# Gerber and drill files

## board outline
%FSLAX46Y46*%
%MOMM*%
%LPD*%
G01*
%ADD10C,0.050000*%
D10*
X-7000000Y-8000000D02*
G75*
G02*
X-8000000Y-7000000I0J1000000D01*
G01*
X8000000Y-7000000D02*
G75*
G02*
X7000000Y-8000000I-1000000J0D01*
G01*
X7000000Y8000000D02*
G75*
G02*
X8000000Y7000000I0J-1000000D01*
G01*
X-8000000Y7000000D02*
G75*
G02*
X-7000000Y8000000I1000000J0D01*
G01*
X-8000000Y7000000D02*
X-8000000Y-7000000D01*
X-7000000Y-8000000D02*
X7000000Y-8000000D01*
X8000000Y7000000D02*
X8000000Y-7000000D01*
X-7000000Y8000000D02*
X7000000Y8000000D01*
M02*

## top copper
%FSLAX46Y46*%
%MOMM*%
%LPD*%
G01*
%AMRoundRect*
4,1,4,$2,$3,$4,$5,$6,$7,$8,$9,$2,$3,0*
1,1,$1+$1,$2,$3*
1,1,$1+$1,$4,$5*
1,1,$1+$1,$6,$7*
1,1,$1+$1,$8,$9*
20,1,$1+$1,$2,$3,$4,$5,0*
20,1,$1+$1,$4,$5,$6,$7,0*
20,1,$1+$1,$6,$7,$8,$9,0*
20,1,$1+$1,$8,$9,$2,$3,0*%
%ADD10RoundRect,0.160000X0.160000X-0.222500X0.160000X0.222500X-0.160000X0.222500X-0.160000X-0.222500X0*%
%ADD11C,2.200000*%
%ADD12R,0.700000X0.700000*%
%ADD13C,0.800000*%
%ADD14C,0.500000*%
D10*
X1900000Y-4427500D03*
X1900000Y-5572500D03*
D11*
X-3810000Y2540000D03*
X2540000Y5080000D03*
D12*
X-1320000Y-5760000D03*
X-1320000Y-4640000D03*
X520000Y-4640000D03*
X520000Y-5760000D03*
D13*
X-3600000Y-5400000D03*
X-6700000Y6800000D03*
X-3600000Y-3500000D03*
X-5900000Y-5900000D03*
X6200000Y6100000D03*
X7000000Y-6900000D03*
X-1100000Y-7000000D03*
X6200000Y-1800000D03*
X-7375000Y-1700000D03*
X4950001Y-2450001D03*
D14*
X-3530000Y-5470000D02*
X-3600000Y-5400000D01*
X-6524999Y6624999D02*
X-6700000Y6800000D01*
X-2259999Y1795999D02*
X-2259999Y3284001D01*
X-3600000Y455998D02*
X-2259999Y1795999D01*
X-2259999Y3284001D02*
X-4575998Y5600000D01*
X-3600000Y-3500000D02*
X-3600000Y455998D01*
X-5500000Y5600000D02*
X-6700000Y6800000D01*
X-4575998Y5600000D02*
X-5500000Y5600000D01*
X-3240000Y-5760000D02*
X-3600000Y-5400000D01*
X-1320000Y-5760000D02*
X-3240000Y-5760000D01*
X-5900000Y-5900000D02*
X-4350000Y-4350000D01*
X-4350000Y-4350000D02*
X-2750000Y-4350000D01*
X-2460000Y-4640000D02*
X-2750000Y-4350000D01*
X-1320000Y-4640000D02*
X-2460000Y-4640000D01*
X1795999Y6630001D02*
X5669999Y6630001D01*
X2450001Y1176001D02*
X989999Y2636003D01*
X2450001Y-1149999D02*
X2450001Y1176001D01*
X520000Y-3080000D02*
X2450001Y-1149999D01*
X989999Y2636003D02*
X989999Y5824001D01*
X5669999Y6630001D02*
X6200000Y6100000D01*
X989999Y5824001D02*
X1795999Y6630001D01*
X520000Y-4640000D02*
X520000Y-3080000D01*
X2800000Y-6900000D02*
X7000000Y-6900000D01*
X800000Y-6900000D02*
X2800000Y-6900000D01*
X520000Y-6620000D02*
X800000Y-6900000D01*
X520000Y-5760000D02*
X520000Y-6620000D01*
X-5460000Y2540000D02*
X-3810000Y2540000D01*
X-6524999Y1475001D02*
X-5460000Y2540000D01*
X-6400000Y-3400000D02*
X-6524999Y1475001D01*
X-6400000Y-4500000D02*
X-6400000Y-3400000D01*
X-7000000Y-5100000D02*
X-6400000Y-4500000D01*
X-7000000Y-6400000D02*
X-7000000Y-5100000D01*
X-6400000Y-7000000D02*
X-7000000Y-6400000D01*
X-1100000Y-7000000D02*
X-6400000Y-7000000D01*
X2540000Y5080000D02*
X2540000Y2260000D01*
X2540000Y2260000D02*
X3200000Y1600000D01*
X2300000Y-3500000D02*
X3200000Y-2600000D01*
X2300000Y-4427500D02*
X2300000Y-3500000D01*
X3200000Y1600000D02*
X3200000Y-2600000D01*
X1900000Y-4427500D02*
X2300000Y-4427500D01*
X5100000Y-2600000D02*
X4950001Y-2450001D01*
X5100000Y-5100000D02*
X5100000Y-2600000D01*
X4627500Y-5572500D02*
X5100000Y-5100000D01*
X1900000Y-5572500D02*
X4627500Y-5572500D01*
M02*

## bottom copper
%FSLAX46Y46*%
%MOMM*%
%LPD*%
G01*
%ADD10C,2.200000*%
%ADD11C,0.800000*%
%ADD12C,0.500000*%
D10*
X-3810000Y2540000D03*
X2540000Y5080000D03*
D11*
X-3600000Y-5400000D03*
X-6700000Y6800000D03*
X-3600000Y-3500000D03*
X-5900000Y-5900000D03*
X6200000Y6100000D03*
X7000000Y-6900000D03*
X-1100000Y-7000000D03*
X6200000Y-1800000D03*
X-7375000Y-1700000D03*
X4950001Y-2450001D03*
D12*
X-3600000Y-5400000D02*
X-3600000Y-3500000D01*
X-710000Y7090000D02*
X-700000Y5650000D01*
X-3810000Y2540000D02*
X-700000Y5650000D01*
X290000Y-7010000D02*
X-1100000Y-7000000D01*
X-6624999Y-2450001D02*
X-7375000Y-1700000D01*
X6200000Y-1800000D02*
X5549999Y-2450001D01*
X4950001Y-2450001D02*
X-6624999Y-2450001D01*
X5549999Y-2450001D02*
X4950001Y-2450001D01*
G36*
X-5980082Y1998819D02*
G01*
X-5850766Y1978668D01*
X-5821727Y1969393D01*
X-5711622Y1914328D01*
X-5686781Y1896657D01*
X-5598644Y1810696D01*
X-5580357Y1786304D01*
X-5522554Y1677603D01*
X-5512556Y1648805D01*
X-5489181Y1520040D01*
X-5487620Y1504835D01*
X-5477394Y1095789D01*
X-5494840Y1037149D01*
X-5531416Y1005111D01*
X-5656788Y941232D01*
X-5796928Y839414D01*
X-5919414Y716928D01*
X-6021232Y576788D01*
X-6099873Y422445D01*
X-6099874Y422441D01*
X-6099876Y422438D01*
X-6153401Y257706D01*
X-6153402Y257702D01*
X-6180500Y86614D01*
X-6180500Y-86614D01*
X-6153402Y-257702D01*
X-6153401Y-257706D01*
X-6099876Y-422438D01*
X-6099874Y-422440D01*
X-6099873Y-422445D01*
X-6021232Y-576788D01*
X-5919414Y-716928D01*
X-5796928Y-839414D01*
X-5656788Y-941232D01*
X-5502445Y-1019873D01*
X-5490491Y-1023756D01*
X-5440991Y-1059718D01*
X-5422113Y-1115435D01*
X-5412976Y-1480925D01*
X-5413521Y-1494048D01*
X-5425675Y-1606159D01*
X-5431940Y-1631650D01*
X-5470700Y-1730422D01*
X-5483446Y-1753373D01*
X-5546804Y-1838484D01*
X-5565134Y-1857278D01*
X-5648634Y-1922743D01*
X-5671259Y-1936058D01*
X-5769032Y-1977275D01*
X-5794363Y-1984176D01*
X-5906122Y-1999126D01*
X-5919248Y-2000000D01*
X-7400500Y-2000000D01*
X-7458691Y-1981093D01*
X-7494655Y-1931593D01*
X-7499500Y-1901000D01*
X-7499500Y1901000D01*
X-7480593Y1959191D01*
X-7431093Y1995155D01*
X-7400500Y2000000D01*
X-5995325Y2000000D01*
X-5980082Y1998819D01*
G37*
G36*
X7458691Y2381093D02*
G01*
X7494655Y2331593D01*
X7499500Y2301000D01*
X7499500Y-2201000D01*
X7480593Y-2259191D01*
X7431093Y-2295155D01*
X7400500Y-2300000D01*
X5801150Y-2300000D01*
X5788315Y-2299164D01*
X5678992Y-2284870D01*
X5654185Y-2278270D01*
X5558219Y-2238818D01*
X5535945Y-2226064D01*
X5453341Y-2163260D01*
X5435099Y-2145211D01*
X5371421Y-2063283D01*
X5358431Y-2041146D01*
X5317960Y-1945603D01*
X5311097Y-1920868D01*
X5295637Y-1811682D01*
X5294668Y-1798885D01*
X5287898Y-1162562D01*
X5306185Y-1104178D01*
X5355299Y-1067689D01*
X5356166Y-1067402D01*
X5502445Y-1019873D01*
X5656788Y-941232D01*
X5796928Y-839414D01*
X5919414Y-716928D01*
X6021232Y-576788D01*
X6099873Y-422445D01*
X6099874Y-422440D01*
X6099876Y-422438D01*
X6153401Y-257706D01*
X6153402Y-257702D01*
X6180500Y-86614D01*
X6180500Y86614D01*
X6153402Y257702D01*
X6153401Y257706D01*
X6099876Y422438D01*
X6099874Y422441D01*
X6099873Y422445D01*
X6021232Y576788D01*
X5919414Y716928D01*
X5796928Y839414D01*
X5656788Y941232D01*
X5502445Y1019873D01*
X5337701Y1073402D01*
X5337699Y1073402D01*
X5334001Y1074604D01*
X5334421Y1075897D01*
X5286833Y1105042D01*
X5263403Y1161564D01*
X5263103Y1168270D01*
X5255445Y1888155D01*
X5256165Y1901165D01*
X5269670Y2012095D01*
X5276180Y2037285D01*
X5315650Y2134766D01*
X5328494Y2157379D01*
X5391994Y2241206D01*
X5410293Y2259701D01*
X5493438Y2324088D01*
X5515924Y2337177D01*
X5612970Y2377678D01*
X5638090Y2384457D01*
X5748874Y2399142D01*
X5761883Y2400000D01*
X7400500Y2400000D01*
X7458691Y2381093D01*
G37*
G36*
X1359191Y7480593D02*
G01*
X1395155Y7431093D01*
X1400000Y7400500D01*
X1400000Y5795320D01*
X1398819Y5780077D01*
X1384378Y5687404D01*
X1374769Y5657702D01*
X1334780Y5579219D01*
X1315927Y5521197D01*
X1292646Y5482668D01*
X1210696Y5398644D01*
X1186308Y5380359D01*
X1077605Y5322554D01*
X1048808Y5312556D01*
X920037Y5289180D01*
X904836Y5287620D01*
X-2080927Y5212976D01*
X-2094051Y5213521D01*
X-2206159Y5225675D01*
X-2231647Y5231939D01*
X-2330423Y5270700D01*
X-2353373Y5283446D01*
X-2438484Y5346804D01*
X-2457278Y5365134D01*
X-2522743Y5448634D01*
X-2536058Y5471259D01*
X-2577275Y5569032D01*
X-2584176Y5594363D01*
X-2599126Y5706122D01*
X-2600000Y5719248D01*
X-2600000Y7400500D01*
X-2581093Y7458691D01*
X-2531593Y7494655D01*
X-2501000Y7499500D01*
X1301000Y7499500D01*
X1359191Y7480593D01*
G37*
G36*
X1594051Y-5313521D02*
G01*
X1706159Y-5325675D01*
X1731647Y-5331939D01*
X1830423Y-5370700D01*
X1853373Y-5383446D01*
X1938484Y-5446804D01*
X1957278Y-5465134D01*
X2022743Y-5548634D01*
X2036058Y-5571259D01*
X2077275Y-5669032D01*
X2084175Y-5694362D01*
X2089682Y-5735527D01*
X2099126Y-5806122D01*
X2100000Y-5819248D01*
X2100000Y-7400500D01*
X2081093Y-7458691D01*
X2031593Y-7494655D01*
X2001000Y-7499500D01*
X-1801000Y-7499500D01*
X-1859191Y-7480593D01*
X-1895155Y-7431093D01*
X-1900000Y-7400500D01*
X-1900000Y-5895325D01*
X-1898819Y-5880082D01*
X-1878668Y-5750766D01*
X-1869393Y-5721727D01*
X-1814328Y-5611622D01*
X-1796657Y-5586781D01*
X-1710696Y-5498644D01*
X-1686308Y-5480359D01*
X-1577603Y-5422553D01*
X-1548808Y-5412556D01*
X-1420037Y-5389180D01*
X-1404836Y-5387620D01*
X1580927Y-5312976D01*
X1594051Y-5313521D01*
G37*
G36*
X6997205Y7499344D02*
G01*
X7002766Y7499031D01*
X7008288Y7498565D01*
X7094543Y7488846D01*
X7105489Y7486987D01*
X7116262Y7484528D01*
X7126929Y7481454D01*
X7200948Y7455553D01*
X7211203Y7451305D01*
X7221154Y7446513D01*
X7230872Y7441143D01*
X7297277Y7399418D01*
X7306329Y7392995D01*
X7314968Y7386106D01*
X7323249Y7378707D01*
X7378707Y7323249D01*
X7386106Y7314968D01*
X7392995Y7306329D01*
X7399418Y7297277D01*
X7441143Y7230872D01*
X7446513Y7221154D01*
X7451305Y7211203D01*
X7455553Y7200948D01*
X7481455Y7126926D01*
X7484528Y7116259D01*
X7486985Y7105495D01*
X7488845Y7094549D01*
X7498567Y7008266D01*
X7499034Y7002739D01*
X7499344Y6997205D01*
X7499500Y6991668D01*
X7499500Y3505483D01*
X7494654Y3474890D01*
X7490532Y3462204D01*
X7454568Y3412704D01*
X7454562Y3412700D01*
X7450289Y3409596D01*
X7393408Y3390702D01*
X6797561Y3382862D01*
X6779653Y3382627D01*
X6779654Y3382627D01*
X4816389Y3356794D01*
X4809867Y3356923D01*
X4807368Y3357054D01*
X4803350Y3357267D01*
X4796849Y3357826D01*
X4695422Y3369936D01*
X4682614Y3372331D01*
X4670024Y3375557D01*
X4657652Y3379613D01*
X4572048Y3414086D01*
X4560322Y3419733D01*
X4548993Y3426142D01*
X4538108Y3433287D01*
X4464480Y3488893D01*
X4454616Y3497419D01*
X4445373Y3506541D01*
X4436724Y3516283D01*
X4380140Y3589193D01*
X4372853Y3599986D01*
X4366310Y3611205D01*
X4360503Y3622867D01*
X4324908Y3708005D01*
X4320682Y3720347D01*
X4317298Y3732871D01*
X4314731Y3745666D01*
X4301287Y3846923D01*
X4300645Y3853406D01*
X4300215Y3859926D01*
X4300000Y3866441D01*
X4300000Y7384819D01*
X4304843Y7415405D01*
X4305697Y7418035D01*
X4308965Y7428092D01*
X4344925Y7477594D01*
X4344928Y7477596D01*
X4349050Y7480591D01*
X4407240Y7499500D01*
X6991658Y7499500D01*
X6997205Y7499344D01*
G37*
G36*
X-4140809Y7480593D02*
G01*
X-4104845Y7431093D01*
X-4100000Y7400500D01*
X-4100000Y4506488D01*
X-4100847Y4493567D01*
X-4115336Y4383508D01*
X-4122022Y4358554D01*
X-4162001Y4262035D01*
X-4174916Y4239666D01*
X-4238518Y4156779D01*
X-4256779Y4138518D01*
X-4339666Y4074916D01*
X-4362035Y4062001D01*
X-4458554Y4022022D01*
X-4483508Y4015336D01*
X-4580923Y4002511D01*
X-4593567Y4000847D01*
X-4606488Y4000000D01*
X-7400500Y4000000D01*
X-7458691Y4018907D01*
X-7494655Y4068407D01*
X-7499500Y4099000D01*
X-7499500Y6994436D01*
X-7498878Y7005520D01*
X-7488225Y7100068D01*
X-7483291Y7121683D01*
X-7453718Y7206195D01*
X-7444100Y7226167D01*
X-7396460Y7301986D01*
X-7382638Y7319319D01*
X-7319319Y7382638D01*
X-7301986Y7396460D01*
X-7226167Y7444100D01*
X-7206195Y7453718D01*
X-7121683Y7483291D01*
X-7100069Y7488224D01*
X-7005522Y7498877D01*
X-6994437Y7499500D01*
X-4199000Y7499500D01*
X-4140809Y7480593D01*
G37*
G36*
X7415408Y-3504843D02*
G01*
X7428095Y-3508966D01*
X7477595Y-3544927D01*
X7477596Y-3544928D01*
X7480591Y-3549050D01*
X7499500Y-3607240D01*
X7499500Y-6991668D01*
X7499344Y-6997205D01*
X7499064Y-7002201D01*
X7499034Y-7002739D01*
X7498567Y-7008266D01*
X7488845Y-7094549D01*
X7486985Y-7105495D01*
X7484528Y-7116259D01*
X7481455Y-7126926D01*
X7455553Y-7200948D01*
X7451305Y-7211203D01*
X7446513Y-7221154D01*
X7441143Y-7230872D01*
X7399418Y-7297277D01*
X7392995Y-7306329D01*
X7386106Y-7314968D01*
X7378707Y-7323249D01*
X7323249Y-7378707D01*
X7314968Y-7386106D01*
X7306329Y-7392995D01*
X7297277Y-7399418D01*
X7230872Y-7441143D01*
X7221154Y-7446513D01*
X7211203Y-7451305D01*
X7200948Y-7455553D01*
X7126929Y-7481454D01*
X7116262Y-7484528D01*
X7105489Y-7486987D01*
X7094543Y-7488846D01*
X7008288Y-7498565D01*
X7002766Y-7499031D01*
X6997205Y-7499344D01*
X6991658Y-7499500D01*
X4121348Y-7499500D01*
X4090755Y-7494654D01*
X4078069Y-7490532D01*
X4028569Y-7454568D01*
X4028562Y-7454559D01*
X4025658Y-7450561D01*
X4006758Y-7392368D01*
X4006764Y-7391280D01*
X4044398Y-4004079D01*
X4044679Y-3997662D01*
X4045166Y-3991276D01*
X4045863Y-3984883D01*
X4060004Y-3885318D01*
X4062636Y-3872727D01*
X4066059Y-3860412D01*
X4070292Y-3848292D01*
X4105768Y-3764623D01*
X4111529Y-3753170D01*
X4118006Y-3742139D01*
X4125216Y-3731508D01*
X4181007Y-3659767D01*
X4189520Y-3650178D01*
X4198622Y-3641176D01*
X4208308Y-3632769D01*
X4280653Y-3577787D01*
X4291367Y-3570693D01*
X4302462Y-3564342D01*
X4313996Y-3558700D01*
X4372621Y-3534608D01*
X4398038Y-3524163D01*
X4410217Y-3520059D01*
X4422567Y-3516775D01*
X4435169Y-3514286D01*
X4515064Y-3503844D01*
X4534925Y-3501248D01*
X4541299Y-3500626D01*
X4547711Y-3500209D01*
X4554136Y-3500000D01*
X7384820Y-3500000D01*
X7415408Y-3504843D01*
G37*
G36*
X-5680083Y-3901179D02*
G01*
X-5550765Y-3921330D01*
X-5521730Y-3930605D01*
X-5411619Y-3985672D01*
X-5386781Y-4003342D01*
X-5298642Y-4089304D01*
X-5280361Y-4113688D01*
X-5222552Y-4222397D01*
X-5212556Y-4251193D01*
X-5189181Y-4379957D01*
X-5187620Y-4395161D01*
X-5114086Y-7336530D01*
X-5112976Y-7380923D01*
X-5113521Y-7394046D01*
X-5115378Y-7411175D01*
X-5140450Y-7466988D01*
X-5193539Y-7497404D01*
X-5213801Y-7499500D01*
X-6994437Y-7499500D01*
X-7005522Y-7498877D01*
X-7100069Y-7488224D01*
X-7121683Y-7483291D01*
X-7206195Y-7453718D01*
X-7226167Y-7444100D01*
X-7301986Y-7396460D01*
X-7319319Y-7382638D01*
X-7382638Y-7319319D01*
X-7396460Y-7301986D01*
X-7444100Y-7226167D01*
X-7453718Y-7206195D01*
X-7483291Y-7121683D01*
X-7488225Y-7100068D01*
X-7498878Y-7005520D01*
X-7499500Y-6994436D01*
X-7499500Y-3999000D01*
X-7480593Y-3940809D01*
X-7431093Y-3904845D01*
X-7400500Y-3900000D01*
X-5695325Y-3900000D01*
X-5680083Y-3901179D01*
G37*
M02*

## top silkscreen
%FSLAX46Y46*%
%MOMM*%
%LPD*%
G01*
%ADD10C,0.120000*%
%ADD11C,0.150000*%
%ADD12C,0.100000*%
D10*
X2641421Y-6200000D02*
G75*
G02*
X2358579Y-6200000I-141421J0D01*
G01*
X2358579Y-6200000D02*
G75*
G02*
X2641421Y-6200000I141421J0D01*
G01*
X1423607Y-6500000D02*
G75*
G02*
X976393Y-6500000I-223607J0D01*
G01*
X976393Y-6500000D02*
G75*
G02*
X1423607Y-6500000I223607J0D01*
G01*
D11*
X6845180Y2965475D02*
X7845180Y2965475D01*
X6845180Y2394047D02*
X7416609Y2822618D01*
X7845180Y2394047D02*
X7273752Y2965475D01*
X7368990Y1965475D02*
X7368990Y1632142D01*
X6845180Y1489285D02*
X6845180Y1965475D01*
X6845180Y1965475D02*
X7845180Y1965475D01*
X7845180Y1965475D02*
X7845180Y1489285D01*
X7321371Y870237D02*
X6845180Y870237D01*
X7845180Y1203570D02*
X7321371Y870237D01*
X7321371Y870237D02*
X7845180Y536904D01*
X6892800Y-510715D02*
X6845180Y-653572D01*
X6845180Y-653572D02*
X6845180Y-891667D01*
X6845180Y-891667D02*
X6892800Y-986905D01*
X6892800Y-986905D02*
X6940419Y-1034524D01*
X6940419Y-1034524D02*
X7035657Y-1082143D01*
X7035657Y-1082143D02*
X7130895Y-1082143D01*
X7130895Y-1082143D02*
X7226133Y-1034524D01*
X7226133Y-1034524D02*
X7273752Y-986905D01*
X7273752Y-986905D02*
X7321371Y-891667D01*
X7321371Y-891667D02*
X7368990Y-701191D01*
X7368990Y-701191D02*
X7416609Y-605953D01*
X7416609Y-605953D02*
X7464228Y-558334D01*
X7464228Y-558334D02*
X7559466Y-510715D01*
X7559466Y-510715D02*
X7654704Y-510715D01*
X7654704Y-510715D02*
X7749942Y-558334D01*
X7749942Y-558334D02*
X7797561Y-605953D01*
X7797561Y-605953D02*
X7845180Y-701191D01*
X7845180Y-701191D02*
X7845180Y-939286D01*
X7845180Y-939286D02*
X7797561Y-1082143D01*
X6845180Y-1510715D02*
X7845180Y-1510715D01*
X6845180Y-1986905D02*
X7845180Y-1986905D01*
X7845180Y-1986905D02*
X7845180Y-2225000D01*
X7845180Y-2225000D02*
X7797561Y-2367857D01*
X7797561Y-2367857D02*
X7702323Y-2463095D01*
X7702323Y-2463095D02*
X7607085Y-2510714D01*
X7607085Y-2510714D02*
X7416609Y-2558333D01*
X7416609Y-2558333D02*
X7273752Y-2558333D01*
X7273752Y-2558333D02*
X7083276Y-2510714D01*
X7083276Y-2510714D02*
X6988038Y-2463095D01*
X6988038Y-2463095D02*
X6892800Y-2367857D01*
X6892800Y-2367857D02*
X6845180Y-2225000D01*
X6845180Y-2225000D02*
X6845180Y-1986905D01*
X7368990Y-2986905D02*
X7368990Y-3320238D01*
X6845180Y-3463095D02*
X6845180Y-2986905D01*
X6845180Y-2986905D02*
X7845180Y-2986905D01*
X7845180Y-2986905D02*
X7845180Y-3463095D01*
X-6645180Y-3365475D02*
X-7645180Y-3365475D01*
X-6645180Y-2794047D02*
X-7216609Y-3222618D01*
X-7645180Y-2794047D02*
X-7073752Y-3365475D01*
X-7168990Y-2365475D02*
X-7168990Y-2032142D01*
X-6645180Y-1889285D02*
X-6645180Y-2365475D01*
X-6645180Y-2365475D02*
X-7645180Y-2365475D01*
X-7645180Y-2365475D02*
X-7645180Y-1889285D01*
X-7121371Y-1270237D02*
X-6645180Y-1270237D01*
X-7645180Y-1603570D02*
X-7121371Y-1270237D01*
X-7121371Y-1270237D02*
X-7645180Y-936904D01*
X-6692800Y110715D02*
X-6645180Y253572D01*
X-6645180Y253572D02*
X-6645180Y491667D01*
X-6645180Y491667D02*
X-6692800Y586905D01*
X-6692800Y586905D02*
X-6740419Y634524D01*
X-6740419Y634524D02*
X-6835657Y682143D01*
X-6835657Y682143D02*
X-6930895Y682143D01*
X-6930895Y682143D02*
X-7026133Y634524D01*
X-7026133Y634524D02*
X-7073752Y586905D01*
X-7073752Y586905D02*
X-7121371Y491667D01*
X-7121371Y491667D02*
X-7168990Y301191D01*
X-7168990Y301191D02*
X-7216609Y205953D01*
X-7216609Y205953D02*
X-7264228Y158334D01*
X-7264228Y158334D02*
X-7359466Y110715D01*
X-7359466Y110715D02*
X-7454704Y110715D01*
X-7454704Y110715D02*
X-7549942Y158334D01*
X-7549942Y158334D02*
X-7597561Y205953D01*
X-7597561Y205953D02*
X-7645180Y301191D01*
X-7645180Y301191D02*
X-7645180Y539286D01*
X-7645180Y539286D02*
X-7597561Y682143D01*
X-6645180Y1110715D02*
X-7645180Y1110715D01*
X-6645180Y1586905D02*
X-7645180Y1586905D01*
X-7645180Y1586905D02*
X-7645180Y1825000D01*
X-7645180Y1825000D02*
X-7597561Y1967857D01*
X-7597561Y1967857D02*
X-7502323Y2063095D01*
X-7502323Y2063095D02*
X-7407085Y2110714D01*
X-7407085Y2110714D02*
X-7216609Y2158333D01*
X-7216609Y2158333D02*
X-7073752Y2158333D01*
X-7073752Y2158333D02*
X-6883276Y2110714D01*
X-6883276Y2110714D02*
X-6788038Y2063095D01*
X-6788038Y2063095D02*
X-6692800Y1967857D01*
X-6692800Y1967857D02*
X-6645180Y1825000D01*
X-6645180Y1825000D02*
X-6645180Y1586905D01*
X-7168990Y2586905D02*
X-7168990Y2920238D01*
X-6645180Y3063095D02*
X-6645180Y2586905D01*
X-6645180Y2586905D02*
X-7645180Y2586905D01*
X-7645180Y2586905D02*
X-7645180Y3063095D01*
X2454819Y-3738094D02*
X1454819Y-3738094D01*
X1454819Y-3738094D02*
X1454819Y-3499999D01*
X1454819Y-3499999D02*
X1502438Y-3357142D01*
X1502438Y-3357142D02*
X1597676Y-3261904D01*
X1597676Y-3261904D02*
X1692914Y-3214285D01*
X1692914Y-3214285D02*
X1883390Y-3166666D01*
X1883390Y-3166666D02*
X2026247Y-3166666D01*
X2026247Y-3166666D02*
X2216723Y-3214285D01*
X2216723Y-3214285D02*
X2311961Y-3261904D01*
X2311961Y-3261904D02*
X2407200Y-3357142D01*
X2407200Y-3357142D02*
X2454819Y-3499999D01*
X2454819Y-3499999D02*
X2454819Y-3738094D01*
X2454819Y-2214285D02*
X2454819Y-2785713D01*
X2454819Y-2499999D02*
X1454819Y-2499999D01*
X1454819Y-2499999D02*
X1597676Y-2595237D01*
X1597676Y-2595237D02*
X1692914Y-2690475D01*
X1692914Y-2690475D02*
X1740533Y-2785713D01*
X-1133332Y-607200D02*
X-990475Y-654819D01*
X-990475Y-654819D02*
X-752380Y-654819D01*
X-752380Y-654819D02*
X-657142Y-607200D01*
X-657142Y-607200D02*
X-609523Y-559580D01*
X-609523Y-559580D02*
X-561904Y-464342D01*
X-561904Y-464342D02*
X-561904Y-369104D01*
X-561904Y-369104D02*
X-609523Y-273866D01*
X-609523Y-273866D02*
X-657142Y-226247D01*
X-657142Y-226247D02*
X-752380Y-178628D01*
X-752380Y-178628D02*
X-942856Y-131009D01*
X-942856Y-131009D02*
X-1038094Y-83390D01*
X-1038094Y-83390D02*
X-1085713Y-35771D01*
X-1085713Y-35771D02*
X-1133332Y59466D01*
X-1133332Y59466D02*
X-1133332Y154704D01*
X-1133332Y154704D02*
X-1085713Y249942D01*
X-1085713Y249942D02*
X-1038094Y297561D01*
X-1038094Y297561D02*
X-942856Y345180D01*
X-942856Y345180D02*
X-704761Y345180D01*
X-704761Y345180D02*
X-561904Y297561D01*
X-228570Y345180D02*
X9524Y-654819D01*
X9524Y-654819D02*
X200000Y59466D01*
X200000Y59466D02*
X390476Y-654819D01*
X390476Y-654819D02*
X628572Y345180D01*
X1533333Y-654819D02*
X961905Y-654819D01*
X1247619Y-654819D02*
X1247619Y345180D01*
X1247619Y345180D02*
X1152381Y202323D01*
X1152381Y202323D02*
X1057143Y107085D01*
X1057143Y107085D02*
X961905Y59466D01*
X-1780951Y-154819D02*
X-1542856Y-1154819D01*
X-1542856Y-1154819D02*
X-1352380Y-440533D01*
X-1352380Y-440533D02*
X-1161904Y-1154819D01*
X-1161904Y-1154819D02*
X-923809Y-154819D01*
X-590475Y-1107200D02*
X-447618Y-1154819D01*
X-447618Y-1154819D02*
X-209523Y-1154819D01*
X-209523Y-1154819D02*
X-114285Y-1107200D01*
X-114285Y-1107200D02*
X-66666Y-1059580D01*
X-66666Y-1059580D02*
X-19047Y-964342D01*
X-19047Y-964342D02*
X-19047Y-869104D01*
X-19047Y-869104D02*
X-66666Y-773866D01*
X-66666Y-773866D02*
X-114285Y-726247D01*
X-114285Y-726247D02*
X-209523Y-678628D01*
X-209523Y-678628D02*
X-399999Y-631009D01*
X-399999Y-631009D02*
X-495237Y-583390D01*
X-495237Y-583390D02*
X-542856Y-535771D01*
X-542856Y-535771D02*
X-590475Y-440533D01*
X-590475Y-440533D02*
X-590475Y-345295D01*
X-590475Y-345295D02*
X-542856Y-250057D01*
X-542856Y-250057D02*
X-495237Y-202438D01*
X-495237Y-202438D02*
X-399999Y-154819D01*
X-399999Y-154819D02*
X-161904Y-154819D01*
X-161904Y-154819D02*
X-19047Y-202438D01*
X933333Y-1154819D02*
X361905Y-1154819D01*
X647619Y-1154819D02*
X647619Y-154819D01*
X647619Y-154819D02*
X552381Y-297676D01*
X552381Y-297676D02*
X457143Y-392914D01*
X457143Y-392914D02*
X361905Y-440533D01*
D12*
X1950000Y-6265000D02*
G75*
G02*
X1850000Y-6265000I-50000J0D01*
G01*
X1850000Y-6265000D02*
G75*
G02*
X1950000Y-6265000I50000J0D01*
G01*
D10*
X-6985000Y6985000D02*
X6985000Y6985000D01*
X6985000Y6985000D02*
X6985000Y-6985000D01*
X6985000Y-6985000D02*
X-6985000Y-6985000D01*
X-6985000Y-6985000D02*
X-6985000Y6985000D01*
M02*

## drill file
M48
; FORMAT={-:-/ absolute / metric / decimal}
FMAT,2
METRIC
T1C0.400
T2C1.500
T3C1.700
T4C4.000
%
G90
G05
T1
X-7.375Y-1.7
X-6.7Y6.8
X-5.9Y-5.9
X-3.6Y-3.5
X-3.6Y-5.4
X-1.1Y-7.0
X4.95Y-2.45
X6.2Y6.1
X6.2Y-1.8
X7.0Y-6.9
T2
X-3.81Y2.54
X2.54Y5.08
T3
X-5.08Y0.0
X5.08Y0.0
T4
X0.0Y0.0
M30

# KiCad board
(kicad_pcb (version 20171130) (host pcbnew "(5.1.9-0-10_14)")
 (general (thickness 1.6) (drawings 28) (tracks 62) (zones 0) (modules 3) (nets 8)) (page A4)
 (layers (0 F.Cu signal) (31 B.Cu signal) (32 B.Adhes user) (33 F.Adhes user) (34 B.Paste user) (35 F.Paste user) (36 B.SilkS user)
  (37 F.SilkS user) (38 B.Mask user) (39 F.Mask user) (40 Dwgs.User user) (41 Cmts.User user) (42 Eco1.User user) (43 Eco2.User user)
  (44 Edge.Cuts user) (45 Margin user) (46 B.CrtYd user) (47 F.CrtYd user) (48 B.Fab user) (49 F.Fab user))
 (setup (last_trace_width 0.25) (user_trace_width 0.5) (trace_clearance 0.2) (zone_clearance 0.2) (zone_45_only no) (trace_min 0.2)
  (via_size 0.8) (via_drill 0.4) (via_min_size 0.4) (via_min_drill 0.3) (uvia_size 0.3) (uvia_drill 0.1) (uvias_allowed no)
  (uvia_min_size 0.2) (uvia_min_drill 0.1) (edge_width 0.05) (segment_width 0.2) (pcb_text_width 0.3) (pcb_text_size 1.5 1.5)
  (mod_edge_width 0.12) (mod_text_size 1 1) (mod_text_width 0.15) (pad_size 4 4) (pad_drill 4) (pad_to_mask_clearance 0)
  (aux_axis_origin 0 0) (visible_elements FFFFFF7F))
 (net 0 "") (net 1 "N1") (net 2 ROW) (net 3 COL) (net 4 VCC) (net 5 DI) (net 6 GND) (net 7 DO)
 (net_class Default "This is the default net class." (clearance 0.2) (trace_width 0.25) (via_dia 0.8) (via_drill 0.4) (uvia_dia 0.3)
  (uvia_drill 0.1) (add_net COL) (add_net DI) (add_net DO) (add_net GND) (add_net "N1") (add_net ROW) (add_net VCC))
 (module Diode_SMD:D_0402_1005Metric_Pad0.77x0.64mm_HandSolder (layer F.Cu) (at 1.9 5 90)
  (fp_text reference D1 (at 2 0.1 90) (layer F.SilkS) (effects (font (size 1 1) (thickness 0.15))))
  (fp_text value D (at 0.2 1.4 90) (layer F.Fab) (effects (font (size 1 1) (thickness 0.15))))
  (fp_circle (center -1.265 0) (end -1.215 0) (layer F.SilkS) (width 0.1))
  (pad 2 smd roundrect (at 0.5725 0 90) (size 0.765 0.64) (layers F.Cu F.Paste F.Mask) (roundrect_rratio 0.25) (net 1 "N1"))
  (pad 1 smd roundrect (at -0.5725 0 90) (size 0.765 0.64) (layers F.Cu F.Paste F.Mask) (roundrect_rratio 0.25) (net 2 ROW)))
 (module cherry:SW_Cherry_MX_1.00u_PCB (layer F.Cu) (at 2.54 -5.08)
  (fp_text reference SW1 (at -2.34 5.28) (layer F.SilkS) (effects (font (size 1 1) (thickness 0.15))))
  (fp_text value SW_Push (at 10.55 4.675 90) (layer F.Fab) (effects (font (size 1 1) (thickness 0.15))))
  (fp_line (start -9.525 -1.905) (end 4.445 -1.905) (layer F.SilkS) (width 0.12))
  (fp_line (start 4.445 -1.905) (end 4.445 12.065) (layer F.SilkS) (width 0.12))
  (fp_line (start 4.445 12.065) (end -9.525 12.065) (layer F.SilkS) (width 0.12))
  (fp_line (start -9.525 12.065) (end -9.525 -1.905) (layer F.SilkS) (width 0.12))
  (pad "" np_thru_hole circle (at 2.54 5.08) (size 1.7 1.7) (drill 1.7) (layers *.Cu *.Mask))
  (pad "" np_thru_hole circle (at -7.62 5.08) (size 1.7 1.7) (drill 1.7) (layers *.Cu *.Mask))
  (pad "" np_thru_hole circle (at -2.54 5.08) (size 4 4) (drill 4) (layers *.Cu *.Mask))
  (pad 2 thru_hole circle (at -6.35 2.54) (size 2.2 2.2) (drill 1.5) (layers *.Cu *.Mask) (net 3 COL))
  (pad 1 thru_hole circle (at 0 0) (size 2.2 2.2) (drill 1.5) (layers *.Cu *.Mask) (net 1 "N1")))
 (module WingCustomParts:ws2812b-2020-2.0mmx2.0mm (layer F.Cu) (at -0.4 5.2)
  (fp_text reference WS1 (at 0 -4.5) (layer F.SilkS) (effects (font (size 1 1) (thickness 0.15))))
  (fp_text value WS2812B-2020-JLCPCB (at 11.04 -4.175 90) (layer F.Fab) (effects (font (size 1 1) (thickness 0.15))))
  (pad 4 smd rect (at -0.92 0.56 180) (size 0.7 0.7) (layers F.Cu F.Paste F.Mask) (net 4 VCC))
  (pad 3 smd rect (at -0.92 -0.56 180) (size 0.7 0.7) (layers F.Cu F.Paste F.Mask) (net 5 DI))
  (pad 2 smd rect (at 0.92 -0.56 180) (size 0.7 0.7) (layers F.Cu F.Paste F.Mask) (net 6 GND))
  (pad 1 smd rect (at 0.92 0.56 180) (size 0.7 0.7) (layers F.Cu F.Paste F.Mask) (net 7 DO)))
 (gr_circle (center 2.5 6.2) (end 2.6 6.3) (layer F.SilkS) (width 0.12))
 (gr_circle (center 1.2 6.5) (end 1.4 6.6) (layer F.SilkS) (width 0.12))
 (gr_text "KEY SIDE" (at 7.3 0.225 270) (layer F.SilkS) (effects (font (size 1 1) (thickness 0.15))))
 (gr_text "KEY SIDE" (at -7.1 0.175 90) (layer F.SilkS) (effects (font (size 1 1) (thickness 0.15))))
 (gr_arc (start -7 7) (end -8 7) (angle -90) (layer Edge.Cuts) (width 0.05))
 (gr_arc (start 7 7) (end 7 8) (angle -90) (layer Edge.Cuts) (width 0.05))
 (gr_arc (start 7 -7) (end 8 -7) (angle -90) (layer Edge.Cuts) (width 0.05))
 (gr_arc (start -7 -7) (end -7 -8) (angle -90) (layer Edge.Cuts) (width 0.05))
 (gr_line (start -8 -7) (end -8 7) (layer Edge.Cuts) (width 0.05))
 (gr_line (start -7 8) (end 7 8) (layer Edge.Cuts) (width 0.05))
 (gr_line (start 8 -7) (end 8 7) (layer Edge.Cuts) (width 0.05))
 (gr_line (start -7 -8) (end 7 -8) (layer Edge.Cuts) (width 0.05))
 (via (at -3.6 5.4) (size 0.8) (drill 0.4) (layers F.Cu B.Cu) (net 4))
 (segment (start -3.53 5.47) (end -3.6 5.4) (width 0.5) (layer F.Cu) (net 4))
 (via (at -6.7 -6.8) (size 0.8) (drill 0.4) (layers F.Cu B.Cu) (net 4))
 (segment (start -6.524999 -6.624999) (end -6.7 -6.8) (width 0.5) (layer F.Cu) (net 4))
 (via (at -3.6 3.5) (size 0.8) (drill 0.4) (layers F.Cu B.Cu) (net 4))
 (segment (start -3.6 5.4) (end -3.6 3.5) (width 0.5) (layer B.Cu) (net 4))
 (segment (start -2.259999 -1.795999) (end -2.259999 -3.284001) (width 0.5) (layer F.Cu) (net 4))
 (segment (start -3.6 -0.455998) (end -2.259999 -1.795999) (width 0.5) (layer F.Cu) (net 4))
 (segment (start -2.259999 -3.284001) (end -4.575998 -5.6) (width 0.5) (layer F.Cu) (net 4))
 (segment (start -3.6 3.5) (end -3.6 -0.455998) (width 0.5) (layer F.Cu) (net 4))
 (segment (start -5.5 -5.6) (end -6.7 -6.8) (width 0.5) (layer F.Cu) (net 4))
 (segment (start -4.575998 -5.6) (end -5.5 -5.6) (width 0.5) (layer F.Cu) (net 4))
 (segment (start -3.24 5.76) (end -3.6 5.4) (width 0.5) (layer F.Cu) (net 4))
 (segment (start -1.32 5.76) (end -3.24 5.76) (width 0.5) (layer F.Cu) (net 4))
 (segment (start -5.9 5.9) (end -4.35 4.35) (width 0.5) (layer F.Cu) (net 5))
 (via (at -5.9 5.9) (size 0.8) (drill 0.4) (layers F.Cu B.Cu) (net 5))
 (segment (start -4.35 4.35) (end -2.75 4.35) (width 0.5) (layer F.Cu) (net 5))
 (segment (start -2.46 4.64) (end -2.75 4.35) (width 0.5) (layer F.Cu) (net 5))
 (segment (start -1.32 4.64) (end -2.46 4.64) (width 0.5) (layer F.Cu) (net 5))
 (via (at 6.2 -6.1) (size 0.8) (drill 0.4) (layers F.Cu B.Cu) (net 6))
 (segment (start 1.795999 -6.630001) (end 5.669999 -6.630001) (width 0.5) (layer F.Cu) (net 6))
 (segment (start 2.450001 -1.176001) (end 0.989999 -2.636003) (width 0.5) (layer F.Cu) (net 6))
 (segment (start 2.450001 1.149999) (end 2.450001 -1.176001) (width 0.5) (layer F.Cu) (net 6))
 (segment (start 0.52 3.08) (end 2.450001 1.149999) (width 0.5) (layer F.Cu) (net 6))
 (segment (start 0.989999 -2.636003) (end 0.989999 -5.824001) (width 0.5) (layer F.Cu) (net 6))
 (segment (start 5.669999 -6.630001) (end 6.2 -6.1) (width 0.5) (layer F.Cu) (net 6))
 (segment (start 0.989999 -5.824001) (end 1.795999 -6.630001) (width 0.5) (layer F.Cu) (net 6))
 (segment (start 0.52 4.64) (end 0.52 3.08) (width 0.5) (layer F.Cu) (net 6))
 (via (at 7 6.9) (size 0.8) (drill 0.4) (layers F.Cu B.Cu) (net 7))
 (segment (start 2.8 6.9) (end 7 6.9) (width 0.5) (layer F.Cu) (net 7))
 (segment (start 0.8 6.9) (end 2.8 6.9) (width 0.5) (layer F.Cu) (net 7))
 (segment (start 0.52 6.62) (end 0.8 6.9) (width 0.5) (layer F.Cu) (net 7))
 (segment (start 0.52 5.76) (end 0.52 6.62) (width 0.5) (layer F.Cu) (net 7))
 (segment (start -0.71 -7.09) (end -0.7 -5.65) (width 0.5) (layer B.Cu) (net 3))
 (segment (start -3.81 -2.54) (end -0.7 -5.65) (width 0.5) (layer B.Cu) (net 3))
 (segment (start -5.46 -2.54) (end -3.81 -2.54) (width 0.5) (layer F.Cu) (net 3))
 (segment (start -6.524999 -1.475001) (end -5.46 -2.54) (width 0.5) (layer F.Cu) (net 3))
 (segment (start -6.4 3.4) (end -6.524999 -1.475001) (width 0.5) (layer F.Cu) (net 3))
 (segment (start -6.4 4.5) (end -6.4 3.4) (width 0.5) (layer F.Cu) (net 3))
 (segment (start -7 5.1) (end -6.4 4.5) (width 0.5) (layer F.Cu) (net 3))
 (segment (start -7 6.4) (end -7 5.1) (width 0.5) (layer F.Cu) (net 3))
 (segment (start -6.4 7) (end -7 6.4) (width 0.5) (layer F.Cu) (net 3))
 (segment (start -1.1 7) (end -6.4 7) (width 0.5) (layer F.Cu) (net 3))
 (segment (start 0.29 7.01) (end -1.1 7) (width 0.5) (layer B.Cu) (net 3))
 (via (at -1.1 7) (size 0.8) (drill 0.4) (layers F.Cu B.Cu) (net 3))
 (segment (start 2.54 -5.08) (end 2.54 -2.26) (width 0.5) (layer F.Cu) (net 1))
 (segment (start 2.54 -2.26) (end 3.2 -1.6) (width 0.5) (layer F.Cu) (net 1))
 (segment (start 2.3 3.5) (end 3.2 2.6) (width 0.5) (layer F.Cu) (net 1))
 (segment (start 2.3 4.4275) (end 2.3 3.5) (width 0.5) (layer F.Cu) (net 1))
 (segment (start 3.2 -1.6) (end 3.2 2.6) (width 0.5) (layer F.Cu) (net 1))
 (segment (start 1.9 4.4275) (end 2.3 4.4275) (width 0.5) (layer F.Cu) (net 1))
 (via (at 6.2 1.8) (size 0.8) (drill 0.4) (layers F.Cu B.Cu) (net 2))
 (via (at -7.375 1.7) (size 0.8) (drill 0.4) (layers F.Cu B.Cu) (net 2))
 (segment (start -6.624999 2.450001) (end -7.375 1.7) (width 0.5) (layer B.Cu) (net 2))
 (segment (start 6.2 1.8) (end 5.549999 2.450001) (width 0.5) (layer B.Cu) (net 2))
 (segment (start 4.950001 2.450001) (end -6.624999 2.450001) (width 0.5) (layer B.Cu) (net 2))
 (segment (start 5.549999 2.450001) (end 4.950001 2.450001) (width 0.5) (layer B.Cu) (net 2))
 (via (at 4.950001 2.450001) (size 0.8) (drill 0.4) (layers F.Cu B.Cu) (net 2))
 (segment (start 5.1 2.6) (end 4.950001 2.450001) (width 0.5) (layer F.Cu) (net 2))
 (segment (start 5.1 5.1) (end 5.1 2.6) (width 0.5) (layer F.Cu) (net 2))
 (segment (start 4.6275 5.5725) (end 5.1 5.1) (width 0.5) (layer F.Cu) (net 2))
 (segment (start 1.9 5.5725) (end 4.6275 5.5725) (width 0.5) (layer F.Cu) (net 2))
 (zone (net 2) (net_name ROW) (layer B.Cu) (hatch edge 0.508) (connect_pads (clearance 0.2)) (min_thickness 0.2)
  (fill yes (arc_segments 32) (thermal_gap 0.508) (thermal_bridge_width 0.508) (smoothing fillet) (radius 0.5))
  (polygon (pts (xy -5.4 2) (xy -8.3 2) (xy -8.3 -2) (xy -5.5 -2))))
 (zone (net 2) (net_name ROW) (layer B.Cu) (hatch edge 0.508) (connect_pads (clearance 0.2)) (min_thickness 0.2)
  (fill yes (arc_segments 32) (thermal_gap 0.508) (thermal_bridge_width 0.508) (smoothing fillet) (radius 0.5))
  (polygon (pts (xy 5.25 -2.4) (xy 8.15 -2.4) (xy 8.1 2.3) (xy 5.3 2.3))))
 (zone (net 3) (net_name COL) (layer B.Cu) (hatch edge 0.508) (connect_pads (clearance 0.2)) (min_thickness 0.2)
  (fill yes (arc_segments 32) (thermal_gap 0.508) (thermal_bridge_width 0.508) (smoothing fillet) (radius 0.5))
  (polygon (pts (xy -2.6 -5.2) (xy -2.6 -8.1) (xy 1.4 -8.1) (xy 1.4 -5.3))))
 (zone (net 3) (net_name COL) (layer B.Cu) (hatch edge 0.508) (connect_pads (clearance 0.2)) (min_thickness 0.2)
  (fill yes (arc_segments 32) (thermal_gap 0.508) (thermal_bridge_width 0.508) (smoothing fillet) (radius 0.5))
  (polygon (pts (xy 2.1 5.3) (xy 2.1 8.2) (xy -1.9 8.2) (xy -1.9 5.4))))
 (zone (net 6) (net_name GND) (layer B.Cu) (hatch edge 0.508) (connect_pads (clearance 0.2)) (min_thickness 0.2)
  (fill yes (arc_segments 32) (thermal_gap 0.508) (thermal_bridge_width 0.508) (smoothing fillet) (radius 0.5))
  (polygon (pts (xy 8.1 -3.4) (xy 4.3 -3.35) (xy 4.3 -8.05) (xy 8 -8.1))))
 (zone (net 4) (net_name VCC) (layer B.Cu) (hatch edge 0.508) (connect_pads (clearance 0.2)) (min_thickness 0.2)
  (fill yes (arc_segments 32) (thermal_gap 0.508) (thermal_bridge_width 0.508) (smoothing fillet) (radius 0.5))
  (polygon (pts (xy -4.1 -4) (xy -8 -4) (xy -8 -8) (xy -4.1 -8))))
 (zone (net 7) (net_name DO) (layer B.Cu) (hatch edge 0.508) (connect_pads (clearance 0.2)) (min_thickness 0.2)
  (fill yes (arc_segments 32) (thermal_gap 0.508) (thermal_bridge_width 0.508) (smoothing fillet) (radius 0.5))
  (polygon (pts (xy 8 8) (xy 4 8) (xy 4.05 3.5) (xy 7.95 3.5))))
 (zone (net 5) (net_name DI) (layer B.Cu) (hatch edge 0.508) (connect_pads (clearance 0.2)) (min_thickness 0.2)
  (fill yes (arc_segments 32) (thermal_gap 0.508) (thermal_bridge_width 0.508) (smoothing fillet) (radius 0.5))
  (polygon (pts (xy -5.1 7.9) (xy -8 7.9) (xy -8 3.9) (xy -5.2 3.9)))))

